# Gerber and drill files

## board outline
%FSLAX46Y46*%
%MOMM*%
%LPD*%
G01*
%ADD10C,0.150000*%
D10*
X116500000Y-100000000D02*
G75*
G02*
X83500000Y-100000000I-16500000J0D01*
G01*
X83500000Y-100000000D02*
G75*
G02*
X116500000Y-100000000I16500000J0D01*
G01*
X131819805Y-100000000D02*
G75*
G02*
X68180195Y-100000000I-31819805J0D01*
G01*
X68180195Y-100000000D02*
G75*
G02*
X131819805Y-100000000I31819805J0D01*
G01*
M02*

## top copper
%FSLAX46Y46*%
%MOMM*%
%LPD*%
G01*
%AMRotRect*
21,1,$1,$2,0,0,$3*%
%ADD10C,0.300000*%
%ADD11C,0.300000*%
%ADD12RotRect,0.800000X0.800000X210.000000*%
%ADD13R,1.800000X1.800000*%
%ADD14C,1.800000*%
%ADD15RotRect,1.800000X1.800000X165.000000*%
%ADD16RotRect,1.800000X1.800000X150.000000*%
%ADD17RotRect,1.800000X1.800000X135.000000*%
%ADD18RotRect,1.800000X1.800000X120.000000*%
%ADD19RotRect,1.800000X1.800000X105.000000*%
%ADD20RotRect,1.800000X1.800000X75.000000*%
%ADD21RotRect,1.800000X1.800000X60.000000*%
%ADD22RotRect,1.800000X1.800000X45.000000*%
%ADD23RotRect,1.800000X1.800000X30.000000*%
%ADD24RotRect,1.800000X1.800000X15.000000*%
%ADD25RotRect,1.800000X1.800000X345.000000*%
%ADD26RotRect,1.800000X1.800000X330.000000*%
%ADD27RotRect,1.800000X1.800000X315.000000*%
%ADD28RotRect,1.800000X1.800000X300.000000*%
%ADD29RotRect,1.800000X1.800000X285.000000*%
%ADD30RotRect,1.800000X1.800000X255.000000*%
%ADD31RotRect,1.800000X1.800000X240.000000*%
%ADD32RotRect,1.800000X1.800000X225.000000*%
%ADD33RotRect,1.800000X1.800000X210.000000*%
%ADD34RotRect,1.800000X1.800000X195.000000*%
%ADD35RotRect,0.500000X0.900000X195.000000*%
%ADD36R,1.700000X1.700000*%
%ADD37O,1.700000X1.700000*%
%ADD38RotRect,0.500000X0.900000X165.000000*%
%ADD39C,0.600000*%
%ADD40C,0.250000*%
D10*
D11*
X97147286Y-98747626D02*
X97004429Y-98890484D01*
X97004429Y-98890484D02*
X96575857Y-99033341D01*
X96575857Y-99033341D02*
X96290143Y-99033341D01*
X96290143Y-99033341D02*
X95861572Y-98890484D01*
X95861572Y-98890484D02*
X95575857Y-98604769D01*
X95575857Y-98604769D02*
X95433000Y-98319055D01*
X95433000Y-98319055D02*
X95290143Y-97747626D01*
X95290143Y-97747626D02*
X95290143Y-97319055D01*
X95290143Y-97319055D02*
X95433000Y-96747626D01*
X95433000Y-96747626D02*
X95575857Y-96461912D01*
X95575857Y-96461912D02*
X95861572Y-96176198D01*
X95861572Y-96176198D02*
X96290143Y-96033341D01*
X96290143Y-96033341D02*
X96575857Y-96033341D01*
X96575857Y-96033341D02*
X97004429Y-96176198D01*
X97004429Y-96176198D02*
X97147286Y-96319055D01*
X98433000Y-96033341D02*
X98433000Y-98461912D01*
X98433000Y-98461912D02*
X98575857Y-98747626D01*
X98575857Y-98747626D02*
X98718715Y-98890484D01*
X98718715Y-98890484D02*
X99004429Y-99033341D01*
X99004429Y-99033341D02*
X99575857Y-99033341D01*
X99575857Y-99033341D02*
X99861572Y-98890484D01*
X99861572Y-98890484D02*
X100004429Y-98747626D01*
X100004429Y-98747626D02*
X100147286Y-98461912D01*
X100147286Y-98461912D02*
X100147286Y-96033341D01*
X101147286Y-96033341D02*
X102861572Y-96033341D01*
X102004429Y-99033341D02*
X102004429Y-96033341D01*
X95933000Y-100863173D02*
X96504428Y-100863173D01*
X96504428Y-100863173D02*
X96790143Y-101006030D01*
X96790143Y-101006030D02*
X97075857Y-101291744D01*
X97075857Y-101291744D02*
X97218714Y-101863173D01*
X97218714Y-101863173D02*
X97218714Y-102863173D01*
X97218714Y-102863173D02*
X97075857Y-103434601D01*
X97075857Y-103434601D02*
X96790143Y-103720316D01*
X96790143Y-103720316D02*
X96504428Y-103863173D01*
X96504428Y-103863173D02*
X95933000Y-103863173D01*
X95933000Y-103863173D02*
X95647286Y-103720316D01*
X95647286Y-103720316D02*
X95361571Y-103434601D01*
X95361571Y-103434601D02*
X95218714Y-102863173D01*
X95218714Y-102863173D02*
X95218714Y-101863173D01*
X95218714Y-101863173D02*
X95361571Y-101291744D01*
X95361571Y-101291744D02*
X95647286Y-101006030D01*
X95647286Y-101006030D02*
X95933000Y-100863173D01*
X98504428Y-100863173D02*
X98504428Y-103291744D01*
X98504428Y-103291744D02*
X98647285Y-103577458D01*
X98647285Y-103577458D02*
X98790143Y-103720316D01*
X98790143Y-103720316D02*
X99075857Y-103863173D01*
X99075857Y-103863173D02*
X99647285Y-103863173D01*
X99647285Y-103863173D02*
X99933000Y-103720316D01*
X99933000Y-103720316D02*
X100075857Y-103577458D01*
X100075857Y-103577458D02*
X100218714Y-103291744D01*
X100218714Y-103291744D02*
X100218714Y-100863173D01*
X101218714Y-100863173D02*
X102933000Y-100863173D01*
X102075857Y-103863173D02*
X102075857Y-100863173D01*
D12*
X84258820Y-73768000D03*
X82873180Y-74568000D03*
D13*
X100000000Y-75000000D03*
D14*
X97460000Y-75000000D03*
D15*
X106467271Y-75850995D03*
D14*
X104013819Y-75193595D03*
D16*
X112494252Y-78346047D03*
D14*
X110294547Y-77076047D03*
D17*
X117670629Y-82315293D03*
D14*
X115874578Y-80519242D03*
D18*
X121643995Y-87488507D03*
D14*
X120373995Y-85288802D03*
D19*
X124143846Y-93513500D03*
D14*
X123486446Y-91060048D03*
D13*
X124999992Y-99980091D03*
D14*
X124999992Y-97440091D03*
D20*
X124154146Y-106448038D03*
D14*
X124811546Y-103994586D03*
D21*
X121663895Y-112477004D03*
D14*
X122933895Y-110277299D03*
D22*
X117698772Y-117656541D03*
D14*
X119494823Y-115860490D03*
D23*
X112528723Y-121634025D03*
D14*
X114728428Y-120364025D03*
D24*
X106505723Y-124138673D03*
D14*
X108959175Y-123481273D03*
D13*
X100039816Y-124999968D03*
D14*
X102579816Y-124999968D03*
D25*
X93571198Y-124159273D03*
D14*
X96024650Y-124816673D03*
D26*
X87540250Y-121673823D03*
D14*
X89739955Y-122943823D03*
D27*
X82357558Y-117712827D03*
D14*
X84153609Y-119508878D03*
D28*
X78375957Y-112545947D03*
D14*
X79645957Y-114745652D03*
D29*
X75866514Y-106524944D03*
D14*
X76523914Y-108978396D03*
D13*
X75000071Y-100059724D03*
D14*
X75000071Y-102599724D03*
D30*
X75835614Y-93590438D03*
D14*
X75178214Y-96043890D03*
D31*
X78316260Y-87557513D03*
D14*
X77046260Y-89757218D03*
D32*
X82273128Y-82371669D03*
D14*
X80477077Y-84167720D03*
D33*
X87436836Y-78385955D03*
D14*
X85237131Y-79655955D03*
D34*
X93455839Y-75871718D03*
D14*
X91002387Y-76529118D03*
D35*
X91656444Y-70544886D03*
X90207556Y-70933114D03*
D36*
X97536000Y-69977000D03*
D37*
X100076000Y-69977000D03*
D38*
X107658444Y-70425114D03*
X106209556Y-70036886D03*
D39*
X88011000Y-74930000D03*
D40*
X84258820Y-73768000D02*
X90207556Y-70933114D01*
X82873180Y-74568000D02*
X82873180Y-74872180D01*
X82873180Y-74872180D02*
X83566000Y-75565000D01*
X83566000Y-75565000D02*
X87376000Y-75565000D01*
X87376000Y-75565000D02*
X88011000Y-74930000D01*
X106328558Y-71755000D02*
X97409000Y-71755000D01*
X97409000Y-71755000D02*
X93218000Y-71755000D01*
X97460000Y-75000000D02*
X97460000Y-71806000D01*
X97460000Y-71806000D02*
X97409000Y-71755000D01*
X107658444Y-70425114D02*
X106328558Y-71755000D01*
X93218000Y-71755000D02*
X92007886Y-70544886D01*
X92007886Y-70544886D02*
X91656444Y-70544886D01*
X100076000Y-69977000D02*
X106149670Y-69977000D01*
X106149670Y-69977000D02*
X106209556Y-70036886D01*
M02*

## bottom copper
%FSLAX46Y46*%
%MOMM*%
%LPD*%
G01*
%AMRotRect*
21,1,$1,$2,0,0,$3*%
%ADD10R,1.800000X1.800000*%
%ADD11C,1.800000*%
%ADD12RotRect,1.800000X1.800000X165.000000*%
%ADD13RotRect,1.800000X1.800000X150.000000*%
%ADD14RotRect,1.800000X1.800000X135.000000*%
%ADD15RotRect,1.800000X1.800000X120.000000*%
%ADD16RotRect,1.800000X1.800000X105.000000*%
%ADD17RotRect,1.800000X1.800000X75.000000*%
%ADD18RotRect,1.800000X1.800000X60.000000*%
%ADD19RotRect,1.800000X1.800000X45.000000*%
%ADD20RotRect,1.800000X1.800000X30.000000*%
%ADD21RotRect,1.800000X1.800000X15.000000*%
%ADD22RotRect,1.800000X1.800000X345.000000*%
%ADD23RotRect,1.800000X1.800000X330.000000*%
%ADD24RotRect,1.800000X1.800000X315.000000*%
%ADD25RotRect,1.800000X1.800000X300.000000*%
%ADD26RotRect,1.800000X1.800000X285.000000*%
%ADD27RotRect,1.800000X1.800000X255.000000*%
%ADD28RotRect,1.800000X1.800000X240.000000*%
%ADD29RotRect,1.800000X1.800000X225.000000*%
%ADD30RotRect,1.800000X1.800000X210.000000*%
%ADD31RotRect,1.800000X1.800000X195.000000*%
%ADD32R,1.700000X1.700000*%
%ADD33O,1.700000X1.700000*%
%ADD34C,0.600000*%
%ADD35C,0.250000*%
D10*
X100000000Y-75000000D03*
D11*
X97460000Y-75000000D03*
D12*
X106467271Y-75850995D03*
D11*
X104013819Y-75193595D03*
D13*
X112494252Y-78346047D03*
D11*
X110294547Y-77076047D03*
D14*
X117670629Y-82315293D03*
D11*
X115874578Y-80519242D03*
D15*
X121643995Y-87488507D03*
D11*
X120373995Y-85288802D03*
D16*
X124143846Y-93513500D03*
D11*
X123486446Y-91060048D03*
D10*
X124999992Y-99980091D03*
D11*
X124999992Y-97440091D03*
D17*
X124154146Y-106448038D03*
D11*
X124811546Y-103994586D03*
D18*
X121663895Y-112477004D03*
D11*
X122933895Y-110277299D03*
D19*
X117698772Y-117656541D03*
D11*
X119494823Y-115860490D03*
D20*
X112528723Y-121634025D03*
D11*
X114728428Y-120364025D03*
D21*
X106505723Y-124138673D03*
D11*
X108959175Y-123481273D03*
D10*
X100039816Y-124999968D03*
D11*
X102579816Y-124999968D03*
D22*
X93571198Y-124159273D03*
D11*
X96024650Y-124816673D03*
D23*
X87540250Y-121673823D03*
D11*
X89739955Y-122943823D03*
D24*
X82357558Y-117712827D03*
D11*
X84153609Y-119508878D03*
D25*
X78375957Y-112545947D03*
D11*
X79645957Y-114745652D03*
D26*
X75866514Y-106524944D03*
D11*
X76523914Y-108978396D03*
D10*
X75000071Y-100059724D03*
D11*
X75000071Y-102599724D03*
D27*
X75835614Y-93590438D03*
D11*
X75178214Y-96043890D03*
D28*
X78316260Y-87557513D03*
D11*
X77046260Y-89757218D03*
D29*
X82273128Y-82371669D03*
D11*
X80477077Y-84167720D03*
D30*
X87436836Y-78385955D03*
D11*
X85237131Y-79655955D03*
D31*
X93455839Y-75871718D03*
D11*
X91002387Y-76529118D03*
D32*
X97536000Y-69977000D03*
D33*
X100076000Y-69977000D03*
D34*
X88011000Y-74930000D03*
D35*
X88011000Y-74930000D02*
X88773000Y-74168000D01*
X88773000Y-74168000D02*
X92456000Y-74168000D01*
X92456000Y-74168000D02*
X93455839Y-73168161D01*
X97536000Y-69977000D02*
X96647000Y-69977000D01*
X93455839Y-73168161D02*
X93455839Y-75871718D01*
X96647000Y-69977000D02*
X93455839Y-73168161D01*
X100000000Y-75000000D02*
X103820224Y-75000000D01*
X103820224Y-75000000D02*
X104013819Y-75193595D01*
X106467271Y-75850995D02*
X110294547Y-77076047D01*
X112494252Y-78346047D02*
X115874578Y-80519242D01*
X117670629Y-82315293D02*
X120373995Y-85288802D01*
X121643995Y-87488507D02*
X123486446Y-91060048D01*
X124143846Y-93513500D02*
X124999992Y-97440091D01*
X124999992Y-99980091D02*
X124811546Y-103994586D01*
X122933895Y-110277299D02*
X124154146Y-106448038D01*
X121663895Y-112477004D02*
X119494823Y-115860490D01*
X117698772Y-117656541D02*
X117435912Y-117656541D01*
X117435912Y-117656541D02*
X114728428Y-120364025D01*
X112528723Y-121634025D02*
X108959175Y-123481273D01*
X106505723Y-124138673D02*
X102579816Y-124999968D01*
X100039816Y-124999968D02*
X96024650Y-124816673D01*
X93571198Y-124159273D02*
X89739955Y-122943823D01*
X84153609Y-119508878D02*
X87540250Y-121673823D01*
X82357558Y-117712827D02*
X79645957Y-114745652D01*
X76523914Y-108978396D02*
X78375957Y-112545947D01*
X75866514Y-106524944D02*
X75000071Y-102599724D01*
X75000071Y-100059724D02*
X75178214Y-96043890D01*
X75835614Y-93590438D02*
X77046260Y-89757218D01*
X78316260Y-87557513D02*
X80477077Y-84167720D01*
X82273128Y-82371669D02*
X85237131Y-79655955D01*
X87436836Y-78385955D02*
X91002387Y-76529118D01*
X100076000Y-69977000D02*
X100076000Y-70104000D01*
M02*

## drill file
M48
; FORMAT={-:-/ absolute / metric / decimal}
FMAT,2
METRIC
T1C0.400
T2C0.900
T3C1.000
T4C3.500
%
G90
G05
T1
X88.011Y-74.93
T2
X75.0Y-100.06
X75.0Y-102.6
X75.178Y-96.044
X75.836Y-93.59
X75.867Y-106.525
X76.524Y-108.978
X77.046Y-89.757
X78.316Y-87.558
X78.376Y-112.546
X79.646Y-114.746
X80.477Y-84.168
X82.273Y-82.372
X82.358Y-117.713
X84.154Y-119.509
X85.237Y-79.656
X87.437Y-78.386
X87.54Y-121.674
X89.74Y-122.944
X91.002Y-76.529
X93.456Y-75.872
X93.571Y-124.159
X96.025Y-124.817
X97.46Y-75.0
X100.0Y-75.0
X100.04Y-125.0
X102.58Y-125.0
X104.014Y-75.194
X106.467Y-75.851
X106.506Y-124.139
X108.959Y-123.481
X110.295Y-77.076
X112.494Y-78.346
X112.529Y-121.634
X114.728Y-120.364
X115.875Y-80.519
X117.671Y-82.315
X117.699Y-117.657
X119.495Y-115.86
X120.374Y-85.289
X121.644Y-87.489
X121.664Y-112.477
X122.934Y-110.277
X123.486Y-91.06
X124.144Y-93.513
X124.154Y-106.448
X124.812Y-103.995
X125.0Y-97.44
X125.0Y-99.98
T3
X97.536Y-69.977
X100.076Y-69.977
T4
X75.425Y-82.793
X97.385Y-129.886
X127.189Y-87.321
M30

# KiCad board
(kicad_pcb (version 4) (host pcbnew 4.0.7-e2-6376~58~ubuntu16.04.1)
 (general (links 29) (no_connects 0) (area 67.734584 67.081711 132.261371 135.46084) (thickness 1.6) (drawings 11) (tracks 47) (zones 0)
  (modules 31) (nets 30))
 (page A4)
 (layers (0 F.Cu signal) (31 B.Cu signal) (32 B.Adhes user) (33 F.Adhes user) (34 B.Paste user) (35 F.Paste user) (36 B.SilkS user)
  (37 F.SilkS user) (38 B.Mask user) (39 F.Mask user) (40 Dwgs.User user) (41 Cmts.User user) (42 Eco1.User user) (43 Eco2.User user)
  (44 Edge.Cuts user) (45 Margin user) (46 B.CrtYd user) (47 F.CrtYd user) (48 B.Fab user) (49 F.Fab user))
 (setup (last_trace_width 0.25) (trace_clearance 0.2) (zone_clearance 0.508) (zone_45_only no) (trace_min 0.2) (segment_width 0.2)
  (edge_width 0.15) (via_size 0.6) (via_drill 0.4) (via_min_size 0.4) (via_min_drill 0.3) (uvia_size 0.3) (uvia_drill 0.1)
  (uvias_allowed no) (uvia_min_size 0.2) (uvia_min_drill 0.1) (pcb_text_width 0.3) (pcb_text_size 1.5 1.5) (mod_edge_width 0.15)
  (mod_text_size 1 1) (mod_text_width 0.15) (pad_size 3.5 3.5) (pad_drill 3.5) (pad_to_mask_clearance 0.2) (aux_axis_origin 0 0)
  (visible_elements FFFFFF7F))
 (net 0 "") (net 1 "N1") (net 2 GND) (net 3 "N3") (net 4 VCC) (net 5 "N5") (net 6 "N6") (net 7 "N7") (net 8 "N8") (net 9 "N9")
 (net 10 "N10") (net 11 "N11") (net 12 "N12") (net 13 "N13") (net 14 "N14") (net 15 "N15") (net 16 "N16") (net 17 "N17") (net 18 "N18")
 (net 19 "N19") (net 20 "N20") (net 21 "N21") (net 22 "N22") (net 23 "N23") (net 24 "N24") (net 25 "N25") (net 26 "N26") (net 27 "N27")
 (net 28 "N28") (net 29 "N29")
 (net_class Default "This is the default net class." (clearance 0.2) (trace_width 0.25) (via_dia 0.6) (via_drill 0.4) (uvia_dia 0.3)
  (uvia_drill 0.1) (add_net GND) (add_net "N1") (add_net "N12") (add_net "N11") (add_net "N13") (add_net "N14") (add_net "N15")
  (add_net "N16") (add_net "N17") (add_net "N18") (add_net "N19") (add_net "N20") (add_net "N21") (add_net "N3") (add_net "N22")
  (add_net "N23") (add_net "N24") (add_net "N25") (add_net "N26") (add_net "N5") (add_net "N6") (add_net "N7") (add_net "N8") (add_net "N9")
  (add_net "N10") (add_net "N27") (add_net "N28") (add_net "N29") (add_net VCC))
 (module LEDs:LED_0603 (layer F.Cu) (at 83.566 74.168 30)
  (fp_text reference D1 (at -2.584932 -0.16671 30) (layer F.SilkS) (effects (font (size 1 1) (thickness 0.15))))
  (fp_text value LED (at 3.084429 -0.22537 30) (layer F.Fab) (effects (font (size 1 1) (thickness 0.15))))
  (pad 2 smd rect (at 0.8 0 210) (size 0.8 0.8) (layers F.Cu F.Paste F.Mask) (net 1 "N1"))
  (pad 1 smd rect (at -0.8 0 210) (size 0.8 0.8) (layers F.Cu F.Paste F.Mask) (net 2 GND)))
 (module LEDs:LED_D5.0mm (layer F.Cu) (at 100 75 180)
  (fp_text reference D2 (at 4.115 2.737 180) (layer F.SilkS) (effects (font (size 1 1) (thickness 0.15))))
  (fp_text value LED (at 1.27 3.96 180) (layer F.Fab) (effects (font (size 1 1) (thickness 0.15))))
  (pad 1 thru_hole rect (at 0 0 180) (size 1.8 1.8) (drill 0.9) (layers *.Cu *.Mask) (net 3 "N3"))
  (pad 2 thru_hole circle (at 2.54 0 180) (size 1.8 1.8) (drill 0.9) (layers *.Cu *.Mask) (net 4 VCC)))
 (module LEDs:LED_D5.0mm (layer F.Cu) (at 106.467271 75.850995 165)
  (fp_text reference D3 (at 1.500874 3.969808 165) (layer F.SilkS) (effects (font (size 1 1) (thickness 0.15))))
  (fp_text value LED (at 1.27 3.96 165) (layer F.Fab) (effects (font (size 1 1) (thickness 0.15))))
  (pad 1 thru_hole rect (at 0 0 165) (size 1.8 1.8) (drill 0.9) (layers *.Cu *.Mask) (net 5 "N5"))
  (pad 2 thru_hole circle (at 2.54 0 165) (size 1.8 1.8) (drill 0.9) (layers *.Cu *.Mask) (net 3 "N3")))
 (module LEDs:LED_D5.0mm (layer F.Cu) (at 112.494252 78.346047 150)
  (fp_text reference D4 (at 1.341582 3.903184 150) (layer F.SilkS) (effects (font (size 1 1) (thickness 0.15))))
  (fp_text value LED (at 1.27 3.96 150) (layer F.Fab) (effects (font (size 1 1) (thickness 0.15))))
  (pad 1 thru_hole rect (at 0 0 150) (size 1.8 1.8) (drill 0.9) (layers *.Cu *.Mask) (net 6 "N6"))
  (pad 2 thru_hole circle (at 2.54 0 150) (size 1.8 1.8) (drill 0.9) (layers *.Cu *.Mask) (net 5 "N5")))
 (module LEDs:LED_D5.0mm (layer F.Cu) (at 117.670629 82.315293 135)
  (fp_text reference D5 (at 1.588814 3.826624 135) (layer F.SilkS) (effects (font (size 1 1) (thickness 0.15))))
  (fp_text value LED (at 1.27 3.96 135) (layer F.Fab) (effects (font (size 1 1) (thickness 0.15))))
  (pad 1 thru_hole rect (at 0 0 135) (size 1.8 1.8) (drill 0.9) (layers *.Cu *.Mask) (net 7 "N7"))
  (pad 2 thru_hole circle (at 2.54 0 135) (size 1.8 1.8) (drill 0.9) (layers *.Cu *.Mask) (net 6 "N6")))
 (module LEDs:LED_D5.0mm (layer F.Cu) (at 121.643995 87.488507 120)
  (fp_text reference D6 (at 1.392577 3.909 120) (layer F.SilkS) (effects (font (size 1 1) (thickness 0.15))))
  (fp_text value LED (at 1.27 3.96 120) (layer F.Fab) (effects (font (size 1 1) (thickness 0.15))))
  (pad 1 thru_hole rect (at 0 0 120) (size 1.8 1.8) (drill 0.9) (layers *.Cu *.Mask) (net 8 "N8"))
  (pad 2 thru_hole circle (at 2.54 0 120) (size 1.8 1.8) (drill 0.9) (layers *.Cu *.Mask) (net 7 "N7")))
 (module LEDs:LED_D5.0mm (layer F.Cu) (at 124.143846 93.5135 105)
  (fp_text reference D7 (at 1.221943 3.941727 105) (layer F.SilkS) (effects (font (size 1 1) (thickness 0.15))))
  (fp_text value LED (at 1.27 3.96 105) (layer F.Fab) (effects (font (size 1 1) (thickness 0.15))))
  (pad 1 thru_hole rect (at 0 0 105) (size 1.8 1.8) (drill 0.9) (layers *.Cu *.Mask) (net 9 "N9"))
  (pad 2 thru_hole circle (at 2.54 0 105) (size 1.8 1.8) (drill 0.9) (layers *.Cu *.Mask) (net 8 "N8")))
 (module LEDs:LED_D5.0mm (layer F.Cu) (at 124.999992 99.980091 90)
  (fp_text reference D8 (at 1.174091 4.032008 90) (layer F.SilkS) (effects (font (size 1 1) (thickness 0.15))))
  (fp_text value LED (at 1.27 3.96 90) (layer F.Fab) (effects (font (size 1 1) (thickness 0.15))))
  (pad 1 thru_hole rect (at 0 0 90) (size 1.8 1.8) (drill 0.9) (layers *.Cu *.Mask) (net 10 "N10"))
  (pad 2 thru_hole circle (at 2.54 0 90) (size 1.8 1.8) (drill 0.9) (layers *.Cu *.Mask) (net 9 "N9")))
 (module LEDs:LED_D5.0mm (layer F.Cu) (at 124.154146 106.448038 75)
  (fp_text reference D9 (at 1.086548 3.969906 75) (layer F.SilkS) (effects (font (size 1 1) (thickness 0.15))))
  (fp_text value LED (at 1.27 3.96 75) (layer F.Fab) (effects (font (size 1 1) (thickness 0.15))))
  (pad 1 thru_hole rect (at 0 0 75) (size 1.8 1.8) (drill 0.9) (layers *.Cu *.Mask) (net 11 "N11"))
  (pad 2 thru_hole circle (at 2.54 0 75) (size 1.8 1.8) (drill 0.9) (layers *.Cu *.Mask) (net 10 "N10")))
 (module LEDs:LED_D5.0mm (layer F.Cu) (at 121.663895 112.477004 60)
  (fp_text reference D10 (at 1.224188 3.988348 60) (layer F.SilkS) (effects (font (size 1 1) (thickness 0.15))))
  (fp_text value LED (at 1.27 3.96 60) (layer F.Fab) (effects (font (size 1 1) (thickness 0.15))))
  (pad 1 thru_hole rect (at 0 0 60) (size 1.8 1.8) (drill 0.9) (layers *.Cu *.Mask) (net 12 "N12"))
  (pad 2 thru_hole circle (at 2.54 0 60) (size 1.8 1.8) (drill 0.9) (layers *.Cu *.Mask) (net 11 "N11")))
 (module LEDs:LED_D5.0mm (layer F.Cu) (at 117.698772 117.656541 45)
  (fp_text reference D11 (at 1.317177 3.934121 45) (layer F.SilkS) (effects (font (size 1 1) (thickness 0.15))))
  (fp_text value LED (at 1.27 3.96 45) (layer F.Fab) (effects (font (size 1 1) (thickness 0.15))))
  (pad 1 thru_hole rect (at 0 0 45) (size 1.8 1.8) (drill 0.9) (layers *.Cu *.Mask) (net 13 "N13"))
  (pad 2 thru_hole circle (at 2.54 0 45) (size 1.8 1.8) (drill 0.9) (layers *.Cu *.Mask) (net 12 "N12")))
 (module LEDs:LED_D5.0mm (layer F.Cu) (at 112.528723 121.634025 30)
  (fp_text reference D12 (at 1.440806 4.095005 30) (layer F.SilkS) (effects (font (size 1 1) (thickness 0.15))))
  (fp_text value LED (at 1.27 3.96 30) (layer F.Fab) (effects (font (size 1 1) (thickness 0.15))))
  (pad 1 thru_hole rect (at 0 0 30) (size 1.8 1.8) (drill 0.9) (layers *.Cu *.Mask) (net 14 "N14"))
  (pad 2 thru_hole circle (at 2.54 0 30) (size 1.8 1.8) (drill 0.9) (layers *.Cu *.Mask) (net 13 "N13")))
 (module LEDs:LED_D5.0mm (layer F.Cu) (at 106.505723 124.138673 15)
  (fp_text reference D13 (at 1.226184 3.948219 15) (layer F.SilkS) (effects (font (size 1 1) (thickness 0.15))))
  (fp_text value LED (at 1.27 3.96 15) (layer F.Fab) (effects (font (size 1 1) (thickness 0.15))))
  (pad 1 thru_hole rect (at 0 0 15) (size 1.8 1.8) (drill 0.9) (layers *.Cu *.Mask) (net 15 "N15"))
  (pad 2 thru_hole circle (at 2.54 0 15) (size 1.8 1.8) (drill 0.9) (layers *.Cu *.Mask) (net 14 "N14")))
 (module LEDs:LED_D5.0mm (layer F.Cu) (at 100.039816 124.999968)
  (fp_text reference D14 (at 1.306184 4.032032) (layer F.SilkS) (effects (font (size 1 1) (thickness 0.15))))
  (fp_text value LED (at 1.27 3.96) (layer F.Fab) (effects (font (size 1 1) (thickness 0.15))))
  (pad 1 thru_hole rect (at 0 0) (size 1.8 1.8) (drill 0.9) (layers *.Cu *.Mask) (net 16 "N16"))
  (pad 2 thru_hole circle (at 2.54 0) (size 1.8 1.8) (drill 0.9) (layers *.Cu *.Mask) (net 15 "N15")))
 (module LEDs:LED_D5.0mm (layer F.Cu) (at 93.571198 124.159273 345)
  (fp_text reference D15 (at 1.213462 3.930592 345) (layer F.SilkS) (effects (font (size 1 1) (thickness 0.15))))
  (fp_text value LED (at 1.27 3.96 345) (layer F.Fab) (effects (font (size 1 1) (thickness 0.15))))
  (pad 1 thru_hole rect (at 0 0 345) (size 1.8 1.8) (drill 0.9) (layers *.Cu *.Mask) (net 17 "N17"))
  (pad 2 thru_hole circle (at 2.54 0 345) (size 1.8 1.8) (drill 0.9) (layers *.Cu *.Mask) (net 16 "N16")))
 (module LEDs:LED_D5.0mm (layer F.Cu) (at 87.54025 121.673823 330)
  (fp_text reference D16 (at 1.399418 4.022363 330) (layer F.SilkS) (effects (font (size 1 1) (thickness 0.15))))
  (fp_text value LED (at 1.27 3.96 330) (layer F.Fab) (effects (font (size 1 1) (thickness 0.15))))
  (pad 1 thru_hole rect (at 0 0 330) (size 1.8 1.8) (drill 0.9) (layers *.Cu *.Mask) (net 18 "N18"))
  (pad 2 thru_hole circle (at 2.54 0 330) (size 1.8 1.8) (drill 0.9) (layers *.Cu *.Mask) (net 17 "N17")))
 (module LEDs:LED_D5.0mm (layer F.Cu) (at 82.357558 117.712827 315)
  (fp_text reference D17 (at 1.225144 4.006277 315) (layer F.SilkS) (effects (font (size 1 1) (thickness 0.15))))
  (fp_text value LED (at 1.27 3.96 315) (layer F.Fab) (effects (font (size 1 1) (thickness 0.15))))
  (pad 1 thru_hole rect (at 0 0 315) (size 1.8 1.8) (drill 0.9) (layers *.Cu *.Mask) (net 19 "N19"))
  (pad 2 thru_hole circle (at 2.54 0 315) (size 1.8 1.8) (drill 0.9) (layers *.Cu *.Mask) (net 18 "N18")))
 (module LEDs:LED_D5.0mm (layer F.Cu) (at 78.375957 112.545947 300)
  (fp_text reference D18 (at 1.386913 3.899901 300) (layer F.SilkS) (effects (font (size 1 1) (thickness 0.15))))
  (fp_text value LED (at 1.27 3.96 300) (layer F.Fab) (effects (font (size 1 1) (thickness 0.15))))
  (pad 1 thru_hole rect (at 0 0 300) (size 1.8 1.8) (drill 0.9) (layers *.Cu *.Mask) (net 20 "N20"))
  (pad 2 thru_hole circle (at 2.54 0 300) (size 1.8 1.8) (drill 0.9) (layers *.Cu *.Mask) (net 19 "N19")))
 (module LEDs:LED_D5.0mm (layer F.Cu) (at 75.866514 106.524944 285)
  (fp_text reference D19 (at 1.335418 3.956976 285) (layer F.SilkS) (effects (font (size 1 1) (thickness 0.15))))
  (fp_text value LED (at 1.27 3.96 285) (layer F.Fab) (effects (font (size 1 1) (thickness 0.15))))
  (pad 1 thru_hole rect (at 0 0 285) (size 1.8 1.8) (drill 0.9) (layers *.Cu *.Mask) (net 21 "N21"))
  (pad 2 thru_hole circle (at 2.54 0 285) (size 1.8 1.8) (drill 0.9) (layers *.Cu *.Mask) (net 20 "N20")))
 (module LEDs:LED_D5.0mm (layer F.Cu) (at 75.000071 100.059724 270)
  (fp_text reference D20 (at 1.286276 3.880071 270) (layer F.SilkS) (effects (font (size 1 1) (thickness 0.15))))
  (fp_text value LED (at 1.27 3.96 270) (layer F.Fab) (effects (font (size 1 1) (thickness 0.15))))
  (pad 1 thru_hole rect (at 0 0 270) (size 1.8 1.8) (drill 0.9) (layers *.Cu *.Mask) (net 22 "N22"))
  (pad 2 thru_hole circle (at 2.54 0 270) (size 1.8 1.8) (drill 0.9) (layers *.Cu *.Mask) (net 21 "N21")))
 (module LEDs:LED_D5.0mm (layer F.Cu) (at 75.835614 93.590438 255)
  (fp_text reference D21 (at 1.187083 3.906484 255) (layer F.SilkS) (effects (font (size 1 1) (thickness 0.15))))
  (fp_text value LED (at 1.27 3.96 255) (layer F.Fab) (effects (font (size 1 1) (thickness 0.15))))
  (pad 1 thru_hole rect (at 0 0 255) (size 1.8 1.8) (drill 0.9) (layers *.Cu *.Mask) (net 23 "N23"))
  (pad 2 thru_hole circle (at 2.54 0 255) (size 1.8 1.8) (drill 0.9) (layers *.Cu *.Mask) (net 22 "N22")))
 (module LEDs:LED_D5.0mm (layer F.Cu) (at 78.31626 87.557513 240)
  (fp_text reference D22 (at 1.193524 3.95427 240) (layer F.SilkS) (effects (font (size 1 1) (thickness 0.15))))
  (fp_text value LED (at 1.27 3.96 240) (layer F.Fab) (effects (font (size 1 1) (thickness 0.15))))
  (pad 1 thru_hole rect (at 0 0 240) (size 1.8 1.8) (drill 0.9) (layers *.Cu *.Mask) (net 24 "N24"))
  (pad 2 thru_hole circle (at 2.54 0 240) (size 1.8 1.8) (drill 0.9) (layers *.Cu *.Mask) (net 23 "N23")))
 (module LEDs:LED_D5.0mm (layer F.Cu) (at 82.273128 82.371669 225)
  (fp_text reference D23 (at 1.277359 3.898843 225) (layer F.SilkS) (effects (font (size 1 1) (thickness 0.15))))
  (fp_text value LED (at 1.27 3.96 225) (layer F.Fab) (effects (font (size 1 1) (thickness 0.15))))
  (pad 1 thru_hole rect (at 0 0 225) (size 1.8 1.8) (drill 0.9) (layers *.Cu *.Mask) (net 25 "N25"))
  (pad 2 thru_hole circle (at 2.54 0 225) (size 1.8 1.8) (drill 0.9) (layers *.Cu *.Mask) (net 24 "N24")))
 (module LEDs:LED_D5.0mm (layer F.Cu) (at 87.436836 78.385955 210)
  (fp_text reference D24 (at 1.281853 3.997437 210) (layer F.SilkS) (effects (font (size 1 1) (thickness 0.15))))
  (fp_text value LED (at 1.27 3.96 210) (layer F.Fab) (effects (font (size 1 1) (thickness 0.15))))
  (pad 1 thru_hole rect (at 0 0 210) (size 1.8 1.8) (drill 0.9) (layers *.Cu *.Mask) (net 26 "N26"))
  (pad 2 thru_hole circle (at 2.54 0 210) (size 1.8 1.8) (drill 0.9) (layers *.Cu *.Mask) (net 25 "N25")))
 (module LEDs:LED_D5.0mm (layer F.Cu) (at 93.455839 75.871718 195)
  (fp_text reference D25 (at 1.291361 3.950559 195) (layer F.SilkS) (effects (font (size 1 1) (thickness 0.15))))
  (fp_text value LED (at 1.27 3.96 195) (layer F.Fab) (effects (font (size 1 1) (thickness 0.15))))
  (pad 1 thru_hole rect (at 0 0 195) (size 1.8 1.8) (drill 0.9) (layers *.Cu *.Mask) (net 2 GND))
  (pad 2 thru_hole circle (at 2.54 0 195) (size 1.8 1.8) (drill 0.9) (layers *.Cu *.Mask) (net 26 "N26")))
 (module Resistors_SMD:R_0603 (layer F.Cu) (at 90.932 70.739 195)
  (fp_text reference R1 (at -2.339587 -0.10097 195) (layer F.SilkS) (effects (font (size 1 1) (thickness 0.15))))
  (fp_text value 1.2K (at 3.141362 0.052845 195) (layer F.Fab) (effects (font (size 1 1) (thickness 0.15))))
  (pad 1 smd rect (at -0.75 0 195) (size 0.5 0.9) (layers F.Cu F.Paste F.Mask) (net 4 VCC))
  (pad 2 smd rect (at 0.75 0 195) (size 0.5 0.9) (layers F.Cu F.Paste F.Mask) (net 1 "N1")))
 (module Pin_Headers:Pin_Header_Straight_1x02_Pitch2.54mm (layer F.Cu) (at 97.536 69.977 90)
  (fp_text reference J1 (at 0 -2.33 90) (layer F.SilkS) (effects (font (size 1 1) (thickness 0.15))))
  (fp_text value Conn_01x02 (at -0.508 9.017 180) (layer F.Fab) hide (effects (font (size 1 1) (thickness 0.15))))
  (pad 1 thru_hole rect (at 0 0 90) (size 1.7 1.7) (drill 1) (layers *.Cu *.Mask) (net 2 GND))
  (pad 2 thru_hole oval (at 0 2.54 90) (size 1.7 1.7) (drill 1) (layers *.Cu *.Mask) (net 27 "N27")))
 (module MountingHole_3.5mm (layer F.Cu) (at 97.385327 129.88584)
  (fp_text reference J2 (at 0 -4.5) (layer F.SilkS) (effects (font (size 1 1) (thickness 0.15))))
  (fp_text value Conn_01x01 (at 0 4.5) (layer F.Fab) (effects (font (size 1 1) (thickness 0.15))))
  (pad 1 np_thru_hole circle (at 0 0) (size 3.5 3.5) (drill 3.5) (layers *.Cu *.Mask) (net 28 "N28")))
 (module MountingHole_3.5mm (layer F.Cu) (at 127.189233 87.321452)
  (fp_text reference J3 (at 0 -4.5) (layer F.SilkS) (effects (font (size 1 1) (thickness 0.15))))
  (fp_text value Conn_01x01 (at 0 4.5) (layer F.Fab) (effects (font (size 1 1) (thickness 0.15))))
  (pad "" np_thru_hole circle (at 0 0) (size 3.5 3.5) (drill 3.5) (layers *.Cu *.Mask)))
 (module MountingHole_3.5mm (layer F.Cu) (at 75.425438 82.792706)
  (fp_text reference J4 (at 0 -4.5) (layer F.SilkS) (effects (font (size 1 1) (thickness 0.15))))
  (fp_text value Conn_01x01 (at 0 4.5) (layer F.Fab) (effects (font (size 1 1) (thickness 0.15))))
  (pad 1 np_thru_hole circle (at 0 0) (size 3.5 3.5) (drill 3.5) (layers *.Cu *.Mask) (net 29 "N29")))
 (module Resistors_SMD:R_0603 (layer F.Cu) (at 106.934 70.231 165)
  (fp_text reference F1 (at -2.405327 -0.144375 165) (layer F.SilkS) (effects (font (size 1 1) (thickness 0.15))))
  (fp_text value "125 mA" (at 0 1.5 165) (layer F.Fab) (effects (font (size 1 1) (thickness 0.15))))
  (pad 1 smd rect (at -0.75 0 165) (size 0.5 0.9) (layers F.Cu F.Paste F.Mask) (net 4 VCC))
  (pad 2 smd rect (at 0.75 0 165) (size 0.5 0.9) (layers F.Cu F.Paste F.Mask) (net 27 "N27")))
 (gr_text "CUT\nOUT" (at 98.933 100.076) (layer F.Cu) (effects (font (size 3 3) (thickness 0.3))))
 (gr_circle (center 100 100) (end 116.5 100) (layer Edge.Cuts) (width 0.15))
 (gr_circle (center 100 100) (end 122.5 122.5) (layer Edge.Cuts) (width 0.15))
 (segment (start 84.25882 73.768) (end 90.207556 70.933114) (width 0.25) (layer F.Cu) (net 1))
 (segment (start 82.87318 74.568) (end 82.87318 74.87218) (width 0.25) (layer F.Cu) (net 2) (status 30))
 (segment (start 82.87318 74.87218) (end 83.566 75.565) (width 0.25) (layer F.Cu) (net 2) (status 10))
 (segment (start 83.566 75.565) (end 87.376 75.565) (width 0.25) (layer F.Cu) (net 2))
 (segment (start 87.376 75.565) (end 88.011 74.93) (width 0.25) (layer F.Cu) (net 2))
 (via (at 88.011 74.93) (size 0.6) (drill 0.4) (layers F.Cu B.Cu) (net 2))
 (segment (start 88.011 74.93) (end 88.773 74.168) (width 0.25) (layer B.Cu) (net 2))
 (segment (start 88.773 74.168) (end 92.456 74.168) (width 0.25) (layer B.Cu) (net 2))
 (segment (start 92.456 74.168) (end 93.455839 73.168161) (width 0.25) (layer B.Cu) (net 2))
 (segment (start 97.536 69.977) (end 96.647 69.977) (width 0.25) (layer B.Cu) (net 2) (status 10))
 (segment (start 93.455839 73.168161) (end 93.455839 75.871718) (width 0.25) (layer B.Cu) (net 2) (status 20))
 (segment (start 96.647 69.977) (end 93.455839 73.168161) (width 0.25) (layer B.Cu) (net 2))
 (segment (start 100 75) (end 103.820224 75) (width 0.25) (layer B.Cu) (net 3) (status 30))
 (segment (start 103.820224 75) (end 104.013819 75.193595) (width 0.25) (layer B.Cu) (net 3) (status 30))
 (segment (start 106.328558 71.755) (end 97.409 71.755) (width 0.25) (layer F.Cu) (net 4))
 (segment (start 97.409 71.755) (end 93.218 71.755) (width 0.25) (layer F.Cu) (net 4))
 (segment (start 97.46 75) (end 97.46 71.806) (width 0.25) (layer F.Cu) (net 4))
 (segment (start 97.46 71.806) (end 97.409 71.755) (width 0.25) (layer F.Cu) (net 4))
 (segment (start 107.658444 70.425114) (end 106.328558 71.755) (width 0.25) (layer F.Cu) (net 4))
 (segment (start 93.218 71.755) (end 92.007886 70.544886) (width 0.25) (layer F.Cu) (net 4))
 (segment (start 92.007886 70.544886) (end 91.656444 70.544886) (width 0.25) (layer F.Cu) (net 4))
 (segment (start 106.467271 75.850995) (end 110.294547 77.076047) (width 0.25) (layer B.Cu) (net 5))
 (segment (start 112.494252 78.346047) (end 115.874578 80.519242) (width 0.25) (layer B.Cu) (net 6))
 (segment (start 117.670629 82.315293) (end 120.373995 85.288802) (width 0.25) (layer B.Cu) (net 7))
 (segment (start 121.643995 87.488507) (end 123.486446 91.060048) (width 0.25) (layer B.Cu) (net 8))
 (segment (start 124.143846 93.5135) (end 124.999992 97.440091) (width 0.25) (layer B.Cu) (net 9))
 (segment (start 124.999992 99.980091) (end 124.811546 103.994586) (width 0.25) (layer B.Cu) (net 10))
 (segment (start 122.933895 110.277299) (end 124.154146 106.448038) (width 0.25) (layer B.Cu) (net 11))
 (segment (start 121.663895 112.477004) (end 119.494823 115.86049) (width 0.25) (layer B.Cu) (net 12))
 (segment (start 117.698772 117.656541) (end 117.435912 117.656541) (width 0.25) (layer B.Cu) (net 13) (status 30))
 (segment (start 117.435912 117.656541) (end 114.728428 120.364025) (width 0.25) (layer B.Cu) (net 13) (status 30))
 (segment (start 112.528723 121.634025) (end 108.959175 123.481273) (width 0.25) (layer B.Cu) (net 14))
 (segment (start 106.505723 124.138673) (end 102.579816 124.999968) (width 0.25) (layer B.Cu) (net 15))
 (segment (start 100.039816 124.999968) (end 96.02465 124.816673) (width 0.25) (layer B.Cu) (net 16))
 (segment (start 93.571198 124.159273) (end 89.739955 122.943823) (width 0.25) (layer B.Cu) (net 17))
 (segment (start 84.153609 119.508878) (end 87.54025 121.673823) (width 0.25) (layer B.Cu) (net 18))
 (segment (start 82.357558 117.712827) (end 79.645957 114.745652) (width 0.25) (layer B.Cu) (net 19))
 (segment (start 76.523914 108.978396) (end 78.375957 112.545947) (width 0.25) (layer B.Cu) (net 20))
 (segment (start 75.866514 106.524944) (end 75.000071 102.599724) (width 0.25) (layer B.Cu) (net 21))
 (segment (start 75.000071 100.059724) (end 75.178214 96.04389) (width 0.25) (layer B.Cu) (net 22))
 (segment (start 75.835614 93.590438) (end 77.04626 89.757218) (width 0.25) (layer B.Cu) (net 23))
 (segment (start 78.31626 87.557513) (end 80.477077 84.16772) (width 0.25) (layer B.Cu) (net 24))
 (segment (start 82.273128 82.371669) (end 85.237131 79.655955) (width 0.25) (layer B.Cu) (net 25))
 (segment (start 87.436836 78.385955) (end 91.002387 76.529118) (width 0.25) (layer B.Cu) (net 26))
 (segment (start 100.076 69.977) (end 106.14967 69.977) (width 0.25) (layer F.Cu) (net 27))
 (segment (start 106.14967 69.977) (end 106.209556 70.036886) (width 0.25) (layer F.Cu) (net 27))
 (segment (start 100.076 69.977) (end 100.076 70.104) (width 0.25) (layer B.Cu) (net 27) (status 30)))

